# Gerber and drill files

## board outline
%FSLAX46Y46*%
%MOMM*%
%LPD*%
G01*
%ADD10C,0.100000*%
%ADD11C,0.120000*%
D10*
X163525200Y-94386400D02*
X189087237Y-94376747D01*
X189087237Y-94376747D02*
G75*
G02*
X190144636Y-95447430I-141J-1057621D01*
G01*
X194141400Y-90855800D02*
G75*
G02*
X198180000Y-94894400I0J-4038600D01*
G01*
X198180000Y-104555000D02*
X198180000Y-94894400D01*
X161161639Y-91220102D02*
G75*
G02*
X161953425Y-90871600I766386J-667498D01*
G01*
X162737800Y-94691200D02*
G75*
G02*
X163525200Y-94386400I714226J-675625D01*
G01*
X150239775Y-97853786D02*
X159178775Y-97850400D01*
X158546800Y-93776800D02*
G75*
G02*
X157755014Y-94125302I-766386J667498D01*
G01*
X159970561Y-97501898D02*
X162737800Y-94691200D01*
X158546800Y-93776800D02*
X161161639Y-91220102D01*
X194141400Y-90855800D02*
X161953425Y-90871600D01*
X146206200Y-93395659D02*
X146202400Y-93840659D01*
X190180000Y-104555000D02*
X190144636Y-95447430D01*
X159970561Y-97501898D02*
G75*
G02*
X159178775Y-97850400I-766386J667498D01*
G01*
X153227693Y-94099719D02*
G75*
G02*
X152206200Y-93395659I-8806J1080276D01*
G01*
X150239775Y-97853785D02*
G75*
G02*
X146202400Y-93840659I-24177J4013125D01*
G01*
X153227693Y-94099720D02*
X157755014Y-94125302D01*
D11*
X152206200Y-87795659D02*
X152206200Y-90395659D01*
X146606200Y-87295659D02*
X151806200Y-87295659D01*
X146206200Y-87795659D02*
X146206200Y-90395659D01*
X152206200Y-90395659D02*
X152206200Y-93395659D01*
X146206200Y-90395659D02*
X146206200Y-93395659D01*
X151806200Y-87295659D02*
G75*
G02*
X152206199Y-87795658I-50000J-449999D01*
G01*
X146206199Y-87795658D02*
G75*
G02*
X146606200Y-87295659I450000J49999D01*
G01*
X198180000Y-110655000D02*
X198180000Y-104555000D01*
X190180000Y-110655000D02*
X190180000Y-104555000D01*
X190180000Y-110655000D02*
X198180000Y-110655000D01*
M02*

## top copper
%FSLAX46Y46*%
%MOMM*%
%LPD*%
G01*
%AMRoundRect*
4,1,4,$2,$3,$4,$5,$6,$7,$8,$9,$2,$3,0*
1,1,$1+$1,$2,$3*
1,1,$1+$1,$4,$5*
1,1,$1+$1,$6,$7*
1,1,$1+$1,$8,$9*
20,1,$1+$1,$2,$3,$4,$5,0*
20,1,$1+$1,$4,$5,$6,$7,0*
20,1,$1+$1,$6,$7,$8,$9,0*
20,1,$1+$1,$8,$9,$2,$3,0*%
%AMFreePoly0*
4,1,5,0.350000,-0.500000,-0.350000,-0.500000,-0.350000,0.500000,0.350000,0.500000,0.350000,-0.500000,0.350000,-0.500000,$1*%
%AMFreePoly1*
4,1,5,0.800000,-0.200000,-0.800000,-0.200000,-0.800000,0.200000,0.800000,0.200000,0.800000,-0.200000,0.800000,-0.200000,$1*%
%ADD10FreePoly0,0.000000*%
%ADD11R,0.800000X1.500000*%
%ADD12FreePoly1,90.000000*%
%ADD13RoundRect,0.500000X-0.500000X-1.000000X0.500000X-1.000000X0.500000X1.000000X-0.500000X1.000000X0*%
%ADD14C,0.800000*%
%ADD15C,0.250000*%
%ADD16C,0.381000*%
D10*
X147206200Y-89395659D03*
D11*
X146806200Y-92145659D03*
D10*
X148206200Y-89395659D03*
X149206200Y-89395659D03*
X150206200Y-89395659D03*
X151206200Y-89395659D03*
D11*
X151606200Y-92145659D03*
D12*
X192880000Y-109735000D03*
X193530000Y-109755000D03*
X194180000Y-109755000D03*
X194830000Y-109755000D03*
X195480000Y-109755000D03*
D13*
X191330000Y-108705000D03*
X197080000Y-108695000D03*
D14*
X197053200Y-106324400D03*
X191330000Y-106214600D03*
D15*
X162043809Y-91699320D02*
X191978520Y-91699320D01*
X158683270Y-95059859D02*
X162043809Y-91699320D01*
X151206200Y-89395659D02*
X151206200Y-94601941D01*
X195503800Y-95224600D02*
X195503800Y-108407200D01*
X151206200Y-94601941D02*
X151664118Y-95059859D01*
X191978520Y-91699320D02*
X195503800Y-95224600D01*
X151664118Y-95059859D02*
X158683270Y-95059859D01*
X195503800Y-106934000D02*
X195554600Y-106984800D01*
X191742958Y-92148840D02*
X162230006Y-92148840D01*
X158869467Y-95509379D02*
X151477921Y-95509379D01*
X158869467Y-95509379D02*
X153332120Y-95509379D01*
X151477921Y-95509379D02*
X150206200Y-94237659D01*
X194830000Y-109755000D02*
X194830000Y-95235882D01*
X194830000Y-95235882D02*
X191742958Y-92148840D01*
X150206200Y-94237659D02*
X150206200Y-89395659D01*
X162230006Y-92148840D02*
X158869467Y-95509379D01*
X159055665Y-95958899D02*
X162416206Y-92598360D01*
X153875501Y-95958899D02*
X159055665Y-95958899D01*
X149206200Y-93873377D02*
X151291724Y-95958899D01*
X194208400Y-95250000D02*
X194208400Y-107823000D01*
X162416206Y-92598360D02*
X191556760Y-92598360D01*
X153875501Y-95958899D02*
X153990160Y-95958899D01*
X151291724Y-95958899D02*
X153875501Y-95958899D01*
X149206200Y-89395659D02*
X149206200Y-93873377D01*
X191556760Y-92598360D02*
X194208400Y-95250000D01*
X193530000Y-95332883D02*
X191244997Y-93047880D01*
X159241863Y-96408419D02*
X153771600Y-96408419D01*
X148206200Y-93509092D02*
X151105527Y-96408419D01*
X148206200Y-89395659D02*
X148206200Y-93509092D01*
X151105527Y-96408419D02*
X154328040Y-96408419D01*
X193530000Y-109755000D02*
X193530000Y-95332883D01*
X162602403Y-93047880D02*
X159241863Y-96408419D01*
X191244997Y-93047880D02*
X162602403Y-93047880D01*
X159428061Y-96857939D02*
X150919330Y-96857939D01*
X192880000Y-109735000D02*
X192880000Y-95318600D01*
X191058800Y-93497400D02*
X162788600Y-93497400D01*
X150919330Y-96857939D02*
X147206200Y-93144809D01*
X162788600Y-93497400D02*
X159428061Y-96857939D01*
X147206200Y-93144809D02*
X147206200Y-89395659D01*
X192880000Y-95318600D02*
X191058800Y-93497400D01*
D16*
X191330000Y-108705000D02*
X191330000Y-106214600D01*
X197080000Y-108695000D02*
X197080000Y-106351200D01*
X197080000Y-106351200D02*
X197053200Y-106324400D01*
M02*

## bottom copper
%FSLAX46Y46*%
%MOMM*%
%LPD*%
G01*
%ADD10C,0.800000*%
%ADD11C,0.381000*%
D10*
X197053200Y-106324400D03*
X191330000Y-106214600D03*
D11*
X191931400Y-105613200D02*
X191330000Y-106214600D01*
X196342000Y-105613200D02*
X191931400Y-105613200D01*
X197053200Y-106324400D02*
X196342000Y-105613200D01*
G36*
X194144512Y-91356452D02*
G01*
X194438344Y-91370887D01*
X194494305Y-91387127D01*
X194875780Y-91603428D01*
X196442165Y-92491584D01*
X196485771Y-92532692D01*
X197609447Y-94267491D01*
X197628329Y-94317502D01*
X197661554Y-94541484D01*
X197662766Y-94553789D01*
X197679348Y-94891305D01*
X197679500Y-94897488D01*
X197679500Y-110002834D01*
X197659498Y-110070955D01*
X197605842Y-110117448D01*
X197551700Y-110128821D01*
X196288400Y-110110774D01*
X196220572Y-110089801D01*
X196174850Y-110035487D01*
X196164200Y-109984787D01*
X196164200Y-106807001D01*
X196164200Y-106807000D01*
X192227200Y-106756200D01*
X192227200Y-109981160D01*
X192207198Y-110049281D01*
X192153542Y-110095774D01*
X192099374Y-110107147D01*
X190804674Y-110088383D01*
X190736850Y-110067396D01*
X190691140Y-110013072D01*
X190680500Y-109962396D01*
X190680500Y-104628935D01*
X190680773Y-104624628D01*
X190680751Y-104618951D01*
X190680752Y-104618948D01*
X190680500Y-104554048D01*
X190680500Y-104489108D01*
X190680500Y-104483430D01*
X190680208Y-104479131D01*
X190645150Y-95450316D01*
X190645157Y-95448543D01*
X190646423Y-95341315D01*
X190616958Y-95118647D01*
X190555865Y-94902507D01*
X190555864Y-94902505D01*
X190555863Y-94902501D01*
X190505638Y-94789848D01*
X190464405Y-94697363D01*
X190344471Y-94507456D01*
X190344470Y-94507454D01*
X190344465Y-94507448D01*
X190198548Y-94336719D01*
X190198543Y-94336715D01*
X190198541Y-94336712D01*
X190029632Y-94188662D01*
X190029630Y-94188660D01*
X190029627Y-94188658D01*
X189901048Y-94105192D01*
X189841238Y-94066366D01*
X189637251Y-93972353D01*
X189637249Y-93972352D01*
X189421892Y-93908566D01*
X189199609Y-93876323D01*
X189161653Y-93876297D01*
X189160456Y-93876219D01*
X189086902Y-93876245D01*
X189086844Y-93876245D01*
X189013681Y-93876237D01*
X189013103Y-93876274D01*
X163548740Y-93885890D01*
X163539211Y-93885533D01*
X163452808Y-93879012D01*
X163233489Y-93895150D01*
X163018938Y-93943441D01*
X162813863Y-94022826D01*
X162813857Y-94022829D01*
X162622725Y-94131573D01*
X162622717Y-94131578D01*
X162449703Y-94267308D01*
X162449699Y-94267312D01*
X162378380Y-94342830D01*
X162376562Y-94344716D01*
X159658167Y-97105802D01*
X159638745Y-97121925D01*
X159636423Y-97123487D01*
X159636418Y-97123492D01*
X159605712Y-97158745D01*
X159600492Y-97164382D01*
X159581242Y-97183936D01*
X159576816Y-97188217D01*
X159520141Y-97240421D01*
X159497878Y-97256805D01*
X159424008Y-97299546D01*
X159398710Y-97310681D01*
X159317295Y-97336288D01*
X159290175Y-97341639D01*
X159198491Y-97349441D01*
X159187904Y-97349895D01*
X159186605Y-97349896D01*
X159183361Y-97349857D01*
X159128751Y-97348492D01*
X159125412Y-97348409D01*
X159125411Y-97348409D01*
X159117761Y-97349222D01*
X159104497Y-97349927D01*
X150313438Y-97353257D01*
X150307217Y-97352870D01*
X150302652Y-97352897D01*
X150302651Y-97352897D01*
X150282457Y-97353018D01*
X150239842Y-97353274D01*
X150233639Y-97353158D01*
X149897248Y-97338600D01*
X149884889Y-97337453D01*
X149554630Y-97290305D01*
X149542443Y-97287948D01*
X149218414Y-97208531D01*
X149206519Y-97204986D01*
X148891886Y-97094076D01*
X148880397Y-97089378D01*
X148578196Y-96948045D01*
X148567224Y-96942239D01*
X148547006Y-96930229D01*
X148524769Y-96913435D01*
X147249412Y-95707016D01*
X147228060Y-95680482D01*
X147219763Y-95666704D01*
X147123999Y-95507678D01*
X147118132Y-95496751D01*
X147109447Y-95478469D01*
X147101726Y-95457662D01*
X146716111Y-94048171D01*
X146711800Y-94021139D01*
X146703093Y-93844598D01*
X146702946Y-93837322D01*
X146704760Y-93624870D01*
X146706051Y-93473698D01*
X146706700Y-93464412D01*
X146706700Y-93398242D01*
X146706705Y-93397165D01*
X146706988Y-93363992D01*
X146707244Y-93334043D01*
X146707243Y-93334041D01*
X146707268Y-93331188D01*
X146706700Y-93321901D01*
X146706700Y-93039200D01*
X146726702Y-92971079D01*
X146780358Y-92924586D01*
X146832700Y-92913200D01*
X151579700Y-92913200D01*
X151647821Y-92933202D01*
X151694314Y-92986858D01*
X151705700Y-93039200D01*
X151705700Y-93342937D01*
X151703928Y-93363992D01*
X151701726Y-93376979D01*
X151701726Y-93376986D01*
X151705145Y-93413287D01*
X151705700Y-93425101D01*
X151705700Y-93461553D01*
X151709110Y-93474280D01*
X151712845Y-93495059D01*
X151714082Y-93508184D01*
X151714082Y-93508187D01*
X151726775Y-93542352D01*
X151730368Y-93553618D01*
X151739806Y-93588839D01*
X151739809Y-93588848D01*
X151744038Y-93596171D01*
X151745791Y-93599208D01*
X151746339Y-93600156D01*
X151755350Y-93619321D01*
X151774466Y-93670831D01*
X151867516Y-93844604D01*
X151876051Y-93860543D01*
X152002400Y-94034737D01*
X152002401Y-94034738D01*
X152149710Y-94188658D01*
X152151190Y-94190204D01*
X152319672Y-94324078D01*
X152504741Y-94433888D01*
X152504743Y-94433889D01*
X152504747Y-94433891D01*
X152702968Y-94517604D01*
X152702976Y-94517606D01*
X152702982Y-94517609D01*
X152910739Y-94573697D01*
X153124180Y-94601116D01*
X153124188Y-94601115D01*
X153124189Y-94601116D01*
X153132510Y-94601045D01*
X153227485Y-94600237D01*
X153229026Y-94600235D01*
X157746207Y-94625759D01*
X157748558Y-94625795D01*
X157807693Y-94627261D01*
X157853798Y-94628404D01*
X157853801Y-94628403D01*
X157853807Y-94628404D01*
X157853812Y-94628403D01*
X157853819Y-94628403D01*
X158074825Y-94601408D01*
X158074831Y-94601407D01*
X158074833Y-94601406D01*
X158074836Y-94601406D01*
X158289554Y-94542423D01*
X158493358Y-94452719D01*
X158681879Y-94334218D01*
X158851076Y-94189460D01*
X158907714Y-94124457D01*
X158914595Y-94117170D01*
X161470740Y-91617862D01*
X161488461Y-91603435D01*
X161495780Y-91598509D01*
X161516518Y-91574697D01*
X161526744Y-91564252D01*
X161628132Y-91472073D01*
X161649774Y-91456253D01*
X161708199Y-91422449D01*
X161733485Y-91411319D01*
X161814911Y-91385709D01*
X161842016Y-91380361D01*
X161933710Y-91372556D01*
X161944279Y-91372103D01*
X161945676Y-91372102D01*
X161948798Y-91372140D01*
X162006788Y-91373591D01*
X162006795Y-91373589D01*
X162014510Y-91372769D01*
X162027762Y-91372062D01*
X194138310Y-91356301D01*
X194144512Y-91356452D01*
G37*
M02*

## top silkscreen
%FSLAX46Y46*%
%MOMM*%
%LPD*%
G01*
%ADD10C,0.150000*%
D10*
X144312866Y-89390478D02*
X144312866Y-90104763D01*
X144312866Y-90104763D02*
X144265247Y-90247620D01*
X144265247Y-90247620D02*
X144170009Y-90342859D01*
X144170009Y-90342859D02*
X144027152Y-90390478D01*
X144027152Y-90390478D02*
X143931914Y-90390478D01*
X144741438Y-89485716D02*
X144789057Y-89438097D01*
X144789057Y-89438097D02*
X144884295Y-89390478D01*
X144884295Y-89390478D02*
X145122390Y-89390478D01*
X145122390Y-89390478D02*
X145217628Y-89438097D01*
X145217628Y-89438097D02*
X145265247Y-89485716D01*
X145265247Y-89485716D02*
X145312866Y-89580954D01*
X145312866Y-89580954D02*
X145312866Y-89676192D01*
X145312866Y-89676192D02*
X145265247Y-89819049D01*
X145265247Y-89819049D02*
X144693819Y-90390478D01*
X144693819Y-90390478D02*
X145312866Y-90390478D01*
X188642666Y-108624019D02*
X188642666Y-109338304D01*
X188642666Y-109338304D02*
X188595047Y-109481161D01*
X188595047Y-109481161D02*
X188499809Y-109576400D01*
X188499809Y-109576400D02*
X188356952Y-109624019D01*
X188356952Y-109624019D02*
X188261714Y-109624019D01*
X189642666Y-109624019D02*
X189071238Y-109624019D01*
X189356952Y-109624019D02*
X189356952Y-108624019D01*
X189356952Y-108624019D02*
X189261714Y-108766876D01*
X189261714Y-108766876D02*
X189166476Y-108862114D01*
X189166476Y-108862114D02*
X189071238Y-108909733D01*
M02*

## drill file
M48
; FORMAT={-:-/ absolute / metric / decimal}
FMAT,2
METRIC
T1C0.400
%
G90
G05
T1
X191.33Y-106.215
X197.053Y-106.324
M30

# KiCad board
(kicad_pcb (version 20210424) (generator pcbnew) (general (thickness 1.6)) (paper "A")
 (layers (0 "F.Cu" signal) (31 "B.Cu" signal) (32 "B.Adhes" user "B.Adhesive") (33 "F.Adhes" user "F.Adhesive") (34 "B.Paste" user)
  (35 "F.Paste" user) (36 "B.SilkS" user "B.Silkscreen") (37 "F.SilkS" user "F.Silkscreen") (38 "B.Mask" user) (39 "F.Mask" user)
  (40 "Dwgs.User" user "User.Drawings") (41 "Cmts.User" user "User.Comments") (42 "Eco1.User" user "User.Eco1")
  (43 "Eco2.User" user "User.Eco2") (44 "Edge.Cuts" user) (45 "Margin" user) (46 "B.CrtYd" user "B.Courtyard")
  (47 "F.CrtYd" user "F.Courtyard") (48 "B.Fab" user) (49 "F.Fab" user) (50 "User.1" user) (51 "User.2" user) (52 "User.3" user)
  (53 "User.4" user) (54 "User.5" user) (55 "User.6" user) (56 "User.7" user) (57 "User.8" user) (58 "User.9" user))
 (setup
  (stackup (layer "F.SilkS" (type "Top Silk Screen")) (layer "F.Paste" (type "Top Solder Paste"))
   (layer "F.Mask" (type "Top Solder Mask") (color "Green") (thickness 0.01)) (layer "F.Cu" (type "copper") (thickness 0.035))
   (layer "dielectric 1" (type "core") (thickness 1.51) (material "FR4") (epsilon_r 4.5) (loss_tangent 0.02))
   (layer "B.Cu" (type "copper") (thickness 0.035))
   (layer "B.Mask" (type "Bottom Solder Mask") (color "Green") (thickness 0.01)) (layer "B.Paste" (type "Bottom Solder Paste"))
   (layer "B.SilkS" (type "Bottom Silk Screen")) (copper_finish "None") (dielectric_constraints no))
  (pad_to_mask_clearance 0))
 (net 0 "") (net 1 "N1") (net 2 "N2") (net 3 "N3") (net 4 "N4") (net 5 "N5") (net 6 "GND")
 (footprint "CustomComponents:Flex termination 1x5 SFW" (layer "F.Cu") (at 149.2062 90.395659)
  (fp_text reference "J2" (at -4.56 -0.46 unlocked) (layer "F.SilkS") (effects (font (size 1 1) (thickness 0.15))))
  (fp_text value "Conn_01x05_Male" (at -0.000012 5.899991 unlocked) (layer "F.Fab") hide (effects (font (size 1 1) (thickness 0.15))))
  (fp_line (start 3 -2.6) (end 3 0) (layer "Edge.Cuts") (width 0.12))
  (fp_line (start -2.6 -3.1) (end 2.6 -3.1) (layer "Edge.Cuts") (width 0.12))
  (fp_line (start -3 -2.6) (end -3 0) (layer "Edge.Cuts") (width 0.12))
  (fp_line (start 3 0) (end 3 3) (layer "Edge.Cuts") (width 0.12))
  (fp_line (start -3 0) (end -3 3) (layer "Edge.Cuts") (width 0.12))
  (fp_arc (start 2.55 -2.650001) (end 2.6 -3.1) (angle 90) (layer "Edge.Cuts") (width 0.12))
  (fp_arc (start -2.550001 -2.65) (end -2.6 -3.1) (angle -90) (layer "Edge.Cuts") (width 0.12))
  (pad "1" connect custom (at -2 -1) (size 0.7 1) (layers "F.Cu" "F.Mask") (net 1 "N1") (options (clearance outline) (anchor rect))
   (primitives))
  (pad "1" connect rect (at -2.4 1.75) (size 0.8 1.5) (layers "F.Cu" "F.Mask") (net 1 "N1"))
  (pad "2" connect custom (at -1 -1) (size 0.7 1) (layers "F.Cu" "F.Mask") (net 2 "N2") (options (clearance outline) (anchor rect))
   (primitives))
  (pad "3" connect custom (at 0 -1) (size 0.7 1) (layers "F.Cu" "F.Mask") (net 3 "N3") (options (clearance outline) (anchor rect))
   (primitives))
  (pad "4" connect custom (at 1 -1) (size 0.7 1) (layers "F.Cu" "F.Mask") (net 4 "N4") (options (clearance outline) (anchor rect))
   (primitives))
  (pad "5" connect custom (at 2 -1) (size 0.7 1) (layers "F.Cu" "F.Mask") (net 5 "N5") (options (clearance outline) (anchor rect))
   (primitives))
  (pad "5" connect rect (at 2.4 1.75) (size 0.8 1.5) (layers "F.Cu" "F.Mask") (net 5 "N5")))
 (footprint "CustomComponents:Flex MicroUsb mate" (layer "F.Cu") (at 194.18 112.555)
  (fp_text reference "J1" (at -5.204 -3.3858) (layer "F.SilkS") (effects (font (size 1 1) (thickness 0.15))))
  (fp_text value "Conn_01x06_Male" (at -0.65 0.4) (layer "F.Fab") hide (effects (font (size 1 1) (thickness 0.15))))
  (fp_line (start 4 -1.9) (end 4 -8) (layer "Edge.Cuts") (width 0.12))
  (fp_line (start -4 -1.9) (end -4 -8) (layer "Edge.Cuts") (width 0.12))
  (fp_line (start -4 -1.9) (end 4 -1.9) (layer "Edge.Cuts") (width 0.12))
  (pad "1" smd custom locked (at -1.3 -2.82 90) (size 1.6 0.4) (layers "F.Cu" "F.Paste" "F.Mask") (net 1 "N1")
   (options (clearance outline) (anchor rect)) (primitives))
  (pad "2" smd custom (at -0.65 -2.8 90) (size 1.6 0.4) (layers "F.Cu" "F.Paste" "F.Mask") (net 2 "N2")
   (options (clearance outline) (anchor rect)) (primitives))
  (pad "3" smd custom (at 0 -2.8 90) (size 1.6 0.4) (layers "F.Cu" "F.Paste" "F.Mask") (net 3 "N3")
   (options (clearance outline) (anchor rect)) (primitives))
  (pad "4" smd custom (at 0.65 -2.8 90) (size 1.6 0.4) (layers "F.Cu" "F.Paste" "F.Mask") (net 4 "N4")
   (options (clearance outline) (anchor rect)) (primitives))
  (pad "5" smd custom (at 1.3 -2.8 90) (size 1.6 0.4) (layers "F.Cu" "F.Paste" "F.Mask") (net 5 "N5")
   (options (clearance outline) (anchor rect)) (primitives))
  (pad "6" smd roundrect locked (at -2.85 -3.85) (size 2 3) (layers "F.Cu" "F.Paste" "F.Mask") (roundrect_rratio 0.25) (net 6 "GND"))
  (pad "6" smd roundrect locked (at 2.9 -3.86) (size 2 3) (layers "F.Cu" "F.Paste" "F.Mask") (roundrect_rratio 0.25) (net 6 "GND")))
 (gr_line (start 163.5252 94.3864) (end 189.087237 94.376747) (layer "Edge.Cuts") (width 0.1))
 (gr_arc (start 189.087096 95.434368) (end 190.144636 95.44743) (angle -90.7) (layer "Edge.Cuts") (width 0.1))
 (gr_arc (start 194.1414 94.8944) (end 198.18 94.8944) (angle -90) (layer "Edge.Cuts") (width 0.1))
 (gr_line (start 198.18 104.555) (end 198.18 94.8944) (layer "Edge.Cuts") (width 0.1))
 (gr_arc (start 161.928025 91.8876) (end 161.953425 90.8716) (angle -50.37728241) (layer "Edge.Cuts") (width 0.1))
 (gr_arc (start 163.452026 95.366825) (end 163.5252 94.3864) (angle -50.85924989) (layer "Edge.Cuts") (width 0.1))
 (gr_line (start 150.239775 97.853786) (end 159.178775 97.8504) (layer "Edge.Cuts") (width 0.1))
 (gr_arc (start 157.780414 93.109302) (end 157.755014 94.125302) (angle -50.37728241) (layer "Edge.Cuts") (width 0.1))
 (gr_line (start 159.970561 97.501898) (end 162.7378 94.6912) (layer "Edge.Cuts") (width 0.1))
 (gr_line (start 158.5468 93.7768) (end 161.161639 91.220102) (layer "Edge.Cuts") (width 0.1))
 (gr_line (start 194.1414 90.8558) (end 161.953425 90.8716) (layer "Edge.Cuts") (width 0.1))
 (gr_line (start 146.2062 93.395659) (end 146.2024 93.840659) (layer "Edge.Cuts") (width 0.1))
 (gr_line (start 190.18 104.555) (end 190.144636 95.44743) (layer "Edge.Cuts") (width 0.1))
 (gr_arc (start 159.204175 96.8344) (end 159.178775 97.8504) (angle -50.37728241) (layer "Edge.Cuts") (width 0.1))
 (gr_arc (start 153.218887 93.019443) (end 152.2062 93.395659) (angle -70.08687296) (layer "Edge.Cuts") (width 0.1))
 (gr_arc (start 150.215598 93.84066) (end 146.2024 93.840659) (angle -90.34518742) (layer "Edge.Cuts") (width 0.1))
 (gr_line (start 153.227693 94.09972) (end 157.755014 94.125302) (layer "Edge.Cuts") (width 0.1))
 (segment (start 162.043809 91.69932) (end 191.97852 91.69932) (width 0.25) (layer "F.Cu") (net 5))
 (segment (start 158.68327 95.059859) (end 162.043809 91.69932) (width 0.25) (layer "F.Cu") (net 5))
 (segment (start 151.2062 89.395659) (end 151.2062 94.601941) (width 0.25) (layer "F.Cu") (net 5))
 (segment (start 195.5038 95.2246) (end 195.5038 108.4072) (width 0.25) (layer "F.Cu") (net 5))
 (segment (start 151.2062 94.601941) (end 151.664118 95.059859) (width 0.25) (layer "F.Cu") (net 5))
 (segment (start 191.97852 91.69932) (end 195.5038 95.2246) (width 0.25) (layer "F.Cu") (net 5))
 (segment (start 151.664118 95.059859) (end 158.68327 95.059859) (width 0.25) (layer "F.Cu") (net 5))
 (segment (start 195.5038 106.934) (end 195.5546 106.9848) (width 0.25) (layer "F.Cu") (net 5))
 (segment (start 191.742958 92.14884) (end 162.230006 92.14884) (width 0.25) (layer "F.Cu") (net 4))
 (segment (start 158.869467 95.509379) (end 151.477921 95.509379) (width 0.25) (layer "F.Cu") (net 4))
 (segment (start 158.869467 95.509379) (end 153.33212 95.509379) (width 0.25) (layer "F.Cu") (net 4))
 (segment (start 151.477921 95.509379) (end 150.2062 94.237659) (width 0.25) (layer "F.Cu") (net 4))
 (segment (start 194.83 109.755) (end 194.83 95.235882) (width 0.25) (layer "F.Cu") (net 4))
 (segment (start 194.83 95.235882) (end 191.742958 92.14884) (width 0.25) (layer "F.Cu") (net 4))
 (segment (start 150.2062 94.237659) (end 150.2062 89.395659) (width 0.25) (layer "F.Cu") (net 4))
 (segment (start 162.230006 92.14884) (end 158.869467 95.509379) (width 0.25) (layer "F.Cu") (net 4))
 (segment (start 159.055665 95.958899) (end 162.416206 92.59836) (width 0.25) (layer "F.Cu") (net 3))
 (segment (start 153.875501 95.958899) (end 159.055665 95.958899) (width 0.25) (layer "F.Cu") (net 3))
 (segment (start 149.2062 93.873377) (end 151.291724 95.958899) (width 0.25) (layer "F.Cu") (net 3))
 (segment (start 194.2084 95.25) (end 194.2084 107.823) (width 0.25) (layer "F.Cu") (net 3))
 (segment (start 162.416206 92.59836) (end 191.55676 92.59836) (width 0.25) (layer "F.Cu") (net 3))
 (segment (start 153.875501 95.958899) (end 153.99016 95.958899) (width 0.25) (layer "F.Cu") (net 3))
 (segment (start 151.291724 95.958899) (end 153.875501 95.958899) (width 0.25) (layer "F.Cu") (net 3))
 (segment (start 149.2062 89.395659) (end 149.2062 93.873377) (width 0.25) (layer "F.Cu") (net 3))
 (segment (start 191.55676 92.59836) (end 194.2084 95.25) (width 0.25) (layer "F.Cu") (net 3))
 (segment (start 193.53 95.332883) (end 191.244997 93.04788) (width 0.25) (layer "F.Cu") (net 2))
 (segment (start 159.241863 96.408419) (end 153.7716 96.408419) (width 0.25) (layer "F.Cu") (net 2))
 (segment (start 148.2062 93.509092) (end 151.105527 96.408419) (width 0.25) (layer "F.Cu") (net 2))
 (segment (start 148.2062 89.395659) (end 148.2062 93.509092) (width 0.25) (layer "F.Cu") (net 2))
 (segment (start 151.105527 96.408419) (end 154.32804 96.408419) (width 0.25) (layer "F.Cu") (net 2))
 (segment (start 193.53 109.755) (end 193.53 95.332883) (width 0.25) (layer "F.Cu") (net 2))
 (segment (start 162.602403 93.04788) (end 159.241863 96.408419) (width 0.25) (layer "F.Cu") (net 2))
 (segment (start 191.244997 93.04788) (end 162.602403 93.04788) (width 0.25) (layer "F.Cu") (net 2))
 (segment (start 159.428061 96.857939) (end 150.91933 96.857939) (width 0.25) (layer "F.Cu") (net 1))
 (segment (start 192.88 109.735) (end 192.88 95.3186) (width 0.25) (layer "F.Cu") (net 1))
 (segment (start 191.0588 93.4974) (end 162.7886 93.4974) (width 0.25) (layer "F.Cu") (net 1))
 (segment (start 150.91933 96.857939) (end 147.2062 93.144809) (width 0.25) (layer "F.Cu") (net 1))
 (segment (start 162.7886 93.4974) (end 159.428061 96.857939) (width 0.25) (layer "F.Cu") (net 1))
 (segment (start 147.2062 93.144809) (end 147.2062 89.395659) (width 0.25) (layer "F.Cu") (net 1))
 (segment (start 192.88 95.3186) (end 191.0588 93.4974) (width 0.25) (layer "F.Cu") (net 1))
 (segment (start 191.33 108.705) (end 191.33 106.2146) (width 0.381) (layer "F.Cu") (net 6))
 (segment (start 197.08 108.695) (end 197.08 106.3512) (width 0.381) (layer "F.Cu") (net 6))
 (segment (start 197.08 106.3512) (end 197.0532 106.3244) (width 0.381) (layer "F.Cu") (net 6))
 (via (at 197.0532 106.3244) (size 0.8) (drill 0.4) (layers "F.Cu" "B.Cu") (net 6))
 (via (at 191.33 106.2146) (size 0.8) (drill 0.4) (layers "F.Cu" "B.Cu") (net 6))
 (segment (start 191.9314 105.6132) (end 191.33 106.2146) (width 0.381) (layer "B.Cu") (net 6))
 (segment (start 196.342 105.6132) (end 191.9314 105.6132) (width 0.381) (layer "B.Cu") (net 6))
 (segment (start 197.0532 106.3244) (end 196.342 105.6132) (width 0.381) (layer "B.Cu") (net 6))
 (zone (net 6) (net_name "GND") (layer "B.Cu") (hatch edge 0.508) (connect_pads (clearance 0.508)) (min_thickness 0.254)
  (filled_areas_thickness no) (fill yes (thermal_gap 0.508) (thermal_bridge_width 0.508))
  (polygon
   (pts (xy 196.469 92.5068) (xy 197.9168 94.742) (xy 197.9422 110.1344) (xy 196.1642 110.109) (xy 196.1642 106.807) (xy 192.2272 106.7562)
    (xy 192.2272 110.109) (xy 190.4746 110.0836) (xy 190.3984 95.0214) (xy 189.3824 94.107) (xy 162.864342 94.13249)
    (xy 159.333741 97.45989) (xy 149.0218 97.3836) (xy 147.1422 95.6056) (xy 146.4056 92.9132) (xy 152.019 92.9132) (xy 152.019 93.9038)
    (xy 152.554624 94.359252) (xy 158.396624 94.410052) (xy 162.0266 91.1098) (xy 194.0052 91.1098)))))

